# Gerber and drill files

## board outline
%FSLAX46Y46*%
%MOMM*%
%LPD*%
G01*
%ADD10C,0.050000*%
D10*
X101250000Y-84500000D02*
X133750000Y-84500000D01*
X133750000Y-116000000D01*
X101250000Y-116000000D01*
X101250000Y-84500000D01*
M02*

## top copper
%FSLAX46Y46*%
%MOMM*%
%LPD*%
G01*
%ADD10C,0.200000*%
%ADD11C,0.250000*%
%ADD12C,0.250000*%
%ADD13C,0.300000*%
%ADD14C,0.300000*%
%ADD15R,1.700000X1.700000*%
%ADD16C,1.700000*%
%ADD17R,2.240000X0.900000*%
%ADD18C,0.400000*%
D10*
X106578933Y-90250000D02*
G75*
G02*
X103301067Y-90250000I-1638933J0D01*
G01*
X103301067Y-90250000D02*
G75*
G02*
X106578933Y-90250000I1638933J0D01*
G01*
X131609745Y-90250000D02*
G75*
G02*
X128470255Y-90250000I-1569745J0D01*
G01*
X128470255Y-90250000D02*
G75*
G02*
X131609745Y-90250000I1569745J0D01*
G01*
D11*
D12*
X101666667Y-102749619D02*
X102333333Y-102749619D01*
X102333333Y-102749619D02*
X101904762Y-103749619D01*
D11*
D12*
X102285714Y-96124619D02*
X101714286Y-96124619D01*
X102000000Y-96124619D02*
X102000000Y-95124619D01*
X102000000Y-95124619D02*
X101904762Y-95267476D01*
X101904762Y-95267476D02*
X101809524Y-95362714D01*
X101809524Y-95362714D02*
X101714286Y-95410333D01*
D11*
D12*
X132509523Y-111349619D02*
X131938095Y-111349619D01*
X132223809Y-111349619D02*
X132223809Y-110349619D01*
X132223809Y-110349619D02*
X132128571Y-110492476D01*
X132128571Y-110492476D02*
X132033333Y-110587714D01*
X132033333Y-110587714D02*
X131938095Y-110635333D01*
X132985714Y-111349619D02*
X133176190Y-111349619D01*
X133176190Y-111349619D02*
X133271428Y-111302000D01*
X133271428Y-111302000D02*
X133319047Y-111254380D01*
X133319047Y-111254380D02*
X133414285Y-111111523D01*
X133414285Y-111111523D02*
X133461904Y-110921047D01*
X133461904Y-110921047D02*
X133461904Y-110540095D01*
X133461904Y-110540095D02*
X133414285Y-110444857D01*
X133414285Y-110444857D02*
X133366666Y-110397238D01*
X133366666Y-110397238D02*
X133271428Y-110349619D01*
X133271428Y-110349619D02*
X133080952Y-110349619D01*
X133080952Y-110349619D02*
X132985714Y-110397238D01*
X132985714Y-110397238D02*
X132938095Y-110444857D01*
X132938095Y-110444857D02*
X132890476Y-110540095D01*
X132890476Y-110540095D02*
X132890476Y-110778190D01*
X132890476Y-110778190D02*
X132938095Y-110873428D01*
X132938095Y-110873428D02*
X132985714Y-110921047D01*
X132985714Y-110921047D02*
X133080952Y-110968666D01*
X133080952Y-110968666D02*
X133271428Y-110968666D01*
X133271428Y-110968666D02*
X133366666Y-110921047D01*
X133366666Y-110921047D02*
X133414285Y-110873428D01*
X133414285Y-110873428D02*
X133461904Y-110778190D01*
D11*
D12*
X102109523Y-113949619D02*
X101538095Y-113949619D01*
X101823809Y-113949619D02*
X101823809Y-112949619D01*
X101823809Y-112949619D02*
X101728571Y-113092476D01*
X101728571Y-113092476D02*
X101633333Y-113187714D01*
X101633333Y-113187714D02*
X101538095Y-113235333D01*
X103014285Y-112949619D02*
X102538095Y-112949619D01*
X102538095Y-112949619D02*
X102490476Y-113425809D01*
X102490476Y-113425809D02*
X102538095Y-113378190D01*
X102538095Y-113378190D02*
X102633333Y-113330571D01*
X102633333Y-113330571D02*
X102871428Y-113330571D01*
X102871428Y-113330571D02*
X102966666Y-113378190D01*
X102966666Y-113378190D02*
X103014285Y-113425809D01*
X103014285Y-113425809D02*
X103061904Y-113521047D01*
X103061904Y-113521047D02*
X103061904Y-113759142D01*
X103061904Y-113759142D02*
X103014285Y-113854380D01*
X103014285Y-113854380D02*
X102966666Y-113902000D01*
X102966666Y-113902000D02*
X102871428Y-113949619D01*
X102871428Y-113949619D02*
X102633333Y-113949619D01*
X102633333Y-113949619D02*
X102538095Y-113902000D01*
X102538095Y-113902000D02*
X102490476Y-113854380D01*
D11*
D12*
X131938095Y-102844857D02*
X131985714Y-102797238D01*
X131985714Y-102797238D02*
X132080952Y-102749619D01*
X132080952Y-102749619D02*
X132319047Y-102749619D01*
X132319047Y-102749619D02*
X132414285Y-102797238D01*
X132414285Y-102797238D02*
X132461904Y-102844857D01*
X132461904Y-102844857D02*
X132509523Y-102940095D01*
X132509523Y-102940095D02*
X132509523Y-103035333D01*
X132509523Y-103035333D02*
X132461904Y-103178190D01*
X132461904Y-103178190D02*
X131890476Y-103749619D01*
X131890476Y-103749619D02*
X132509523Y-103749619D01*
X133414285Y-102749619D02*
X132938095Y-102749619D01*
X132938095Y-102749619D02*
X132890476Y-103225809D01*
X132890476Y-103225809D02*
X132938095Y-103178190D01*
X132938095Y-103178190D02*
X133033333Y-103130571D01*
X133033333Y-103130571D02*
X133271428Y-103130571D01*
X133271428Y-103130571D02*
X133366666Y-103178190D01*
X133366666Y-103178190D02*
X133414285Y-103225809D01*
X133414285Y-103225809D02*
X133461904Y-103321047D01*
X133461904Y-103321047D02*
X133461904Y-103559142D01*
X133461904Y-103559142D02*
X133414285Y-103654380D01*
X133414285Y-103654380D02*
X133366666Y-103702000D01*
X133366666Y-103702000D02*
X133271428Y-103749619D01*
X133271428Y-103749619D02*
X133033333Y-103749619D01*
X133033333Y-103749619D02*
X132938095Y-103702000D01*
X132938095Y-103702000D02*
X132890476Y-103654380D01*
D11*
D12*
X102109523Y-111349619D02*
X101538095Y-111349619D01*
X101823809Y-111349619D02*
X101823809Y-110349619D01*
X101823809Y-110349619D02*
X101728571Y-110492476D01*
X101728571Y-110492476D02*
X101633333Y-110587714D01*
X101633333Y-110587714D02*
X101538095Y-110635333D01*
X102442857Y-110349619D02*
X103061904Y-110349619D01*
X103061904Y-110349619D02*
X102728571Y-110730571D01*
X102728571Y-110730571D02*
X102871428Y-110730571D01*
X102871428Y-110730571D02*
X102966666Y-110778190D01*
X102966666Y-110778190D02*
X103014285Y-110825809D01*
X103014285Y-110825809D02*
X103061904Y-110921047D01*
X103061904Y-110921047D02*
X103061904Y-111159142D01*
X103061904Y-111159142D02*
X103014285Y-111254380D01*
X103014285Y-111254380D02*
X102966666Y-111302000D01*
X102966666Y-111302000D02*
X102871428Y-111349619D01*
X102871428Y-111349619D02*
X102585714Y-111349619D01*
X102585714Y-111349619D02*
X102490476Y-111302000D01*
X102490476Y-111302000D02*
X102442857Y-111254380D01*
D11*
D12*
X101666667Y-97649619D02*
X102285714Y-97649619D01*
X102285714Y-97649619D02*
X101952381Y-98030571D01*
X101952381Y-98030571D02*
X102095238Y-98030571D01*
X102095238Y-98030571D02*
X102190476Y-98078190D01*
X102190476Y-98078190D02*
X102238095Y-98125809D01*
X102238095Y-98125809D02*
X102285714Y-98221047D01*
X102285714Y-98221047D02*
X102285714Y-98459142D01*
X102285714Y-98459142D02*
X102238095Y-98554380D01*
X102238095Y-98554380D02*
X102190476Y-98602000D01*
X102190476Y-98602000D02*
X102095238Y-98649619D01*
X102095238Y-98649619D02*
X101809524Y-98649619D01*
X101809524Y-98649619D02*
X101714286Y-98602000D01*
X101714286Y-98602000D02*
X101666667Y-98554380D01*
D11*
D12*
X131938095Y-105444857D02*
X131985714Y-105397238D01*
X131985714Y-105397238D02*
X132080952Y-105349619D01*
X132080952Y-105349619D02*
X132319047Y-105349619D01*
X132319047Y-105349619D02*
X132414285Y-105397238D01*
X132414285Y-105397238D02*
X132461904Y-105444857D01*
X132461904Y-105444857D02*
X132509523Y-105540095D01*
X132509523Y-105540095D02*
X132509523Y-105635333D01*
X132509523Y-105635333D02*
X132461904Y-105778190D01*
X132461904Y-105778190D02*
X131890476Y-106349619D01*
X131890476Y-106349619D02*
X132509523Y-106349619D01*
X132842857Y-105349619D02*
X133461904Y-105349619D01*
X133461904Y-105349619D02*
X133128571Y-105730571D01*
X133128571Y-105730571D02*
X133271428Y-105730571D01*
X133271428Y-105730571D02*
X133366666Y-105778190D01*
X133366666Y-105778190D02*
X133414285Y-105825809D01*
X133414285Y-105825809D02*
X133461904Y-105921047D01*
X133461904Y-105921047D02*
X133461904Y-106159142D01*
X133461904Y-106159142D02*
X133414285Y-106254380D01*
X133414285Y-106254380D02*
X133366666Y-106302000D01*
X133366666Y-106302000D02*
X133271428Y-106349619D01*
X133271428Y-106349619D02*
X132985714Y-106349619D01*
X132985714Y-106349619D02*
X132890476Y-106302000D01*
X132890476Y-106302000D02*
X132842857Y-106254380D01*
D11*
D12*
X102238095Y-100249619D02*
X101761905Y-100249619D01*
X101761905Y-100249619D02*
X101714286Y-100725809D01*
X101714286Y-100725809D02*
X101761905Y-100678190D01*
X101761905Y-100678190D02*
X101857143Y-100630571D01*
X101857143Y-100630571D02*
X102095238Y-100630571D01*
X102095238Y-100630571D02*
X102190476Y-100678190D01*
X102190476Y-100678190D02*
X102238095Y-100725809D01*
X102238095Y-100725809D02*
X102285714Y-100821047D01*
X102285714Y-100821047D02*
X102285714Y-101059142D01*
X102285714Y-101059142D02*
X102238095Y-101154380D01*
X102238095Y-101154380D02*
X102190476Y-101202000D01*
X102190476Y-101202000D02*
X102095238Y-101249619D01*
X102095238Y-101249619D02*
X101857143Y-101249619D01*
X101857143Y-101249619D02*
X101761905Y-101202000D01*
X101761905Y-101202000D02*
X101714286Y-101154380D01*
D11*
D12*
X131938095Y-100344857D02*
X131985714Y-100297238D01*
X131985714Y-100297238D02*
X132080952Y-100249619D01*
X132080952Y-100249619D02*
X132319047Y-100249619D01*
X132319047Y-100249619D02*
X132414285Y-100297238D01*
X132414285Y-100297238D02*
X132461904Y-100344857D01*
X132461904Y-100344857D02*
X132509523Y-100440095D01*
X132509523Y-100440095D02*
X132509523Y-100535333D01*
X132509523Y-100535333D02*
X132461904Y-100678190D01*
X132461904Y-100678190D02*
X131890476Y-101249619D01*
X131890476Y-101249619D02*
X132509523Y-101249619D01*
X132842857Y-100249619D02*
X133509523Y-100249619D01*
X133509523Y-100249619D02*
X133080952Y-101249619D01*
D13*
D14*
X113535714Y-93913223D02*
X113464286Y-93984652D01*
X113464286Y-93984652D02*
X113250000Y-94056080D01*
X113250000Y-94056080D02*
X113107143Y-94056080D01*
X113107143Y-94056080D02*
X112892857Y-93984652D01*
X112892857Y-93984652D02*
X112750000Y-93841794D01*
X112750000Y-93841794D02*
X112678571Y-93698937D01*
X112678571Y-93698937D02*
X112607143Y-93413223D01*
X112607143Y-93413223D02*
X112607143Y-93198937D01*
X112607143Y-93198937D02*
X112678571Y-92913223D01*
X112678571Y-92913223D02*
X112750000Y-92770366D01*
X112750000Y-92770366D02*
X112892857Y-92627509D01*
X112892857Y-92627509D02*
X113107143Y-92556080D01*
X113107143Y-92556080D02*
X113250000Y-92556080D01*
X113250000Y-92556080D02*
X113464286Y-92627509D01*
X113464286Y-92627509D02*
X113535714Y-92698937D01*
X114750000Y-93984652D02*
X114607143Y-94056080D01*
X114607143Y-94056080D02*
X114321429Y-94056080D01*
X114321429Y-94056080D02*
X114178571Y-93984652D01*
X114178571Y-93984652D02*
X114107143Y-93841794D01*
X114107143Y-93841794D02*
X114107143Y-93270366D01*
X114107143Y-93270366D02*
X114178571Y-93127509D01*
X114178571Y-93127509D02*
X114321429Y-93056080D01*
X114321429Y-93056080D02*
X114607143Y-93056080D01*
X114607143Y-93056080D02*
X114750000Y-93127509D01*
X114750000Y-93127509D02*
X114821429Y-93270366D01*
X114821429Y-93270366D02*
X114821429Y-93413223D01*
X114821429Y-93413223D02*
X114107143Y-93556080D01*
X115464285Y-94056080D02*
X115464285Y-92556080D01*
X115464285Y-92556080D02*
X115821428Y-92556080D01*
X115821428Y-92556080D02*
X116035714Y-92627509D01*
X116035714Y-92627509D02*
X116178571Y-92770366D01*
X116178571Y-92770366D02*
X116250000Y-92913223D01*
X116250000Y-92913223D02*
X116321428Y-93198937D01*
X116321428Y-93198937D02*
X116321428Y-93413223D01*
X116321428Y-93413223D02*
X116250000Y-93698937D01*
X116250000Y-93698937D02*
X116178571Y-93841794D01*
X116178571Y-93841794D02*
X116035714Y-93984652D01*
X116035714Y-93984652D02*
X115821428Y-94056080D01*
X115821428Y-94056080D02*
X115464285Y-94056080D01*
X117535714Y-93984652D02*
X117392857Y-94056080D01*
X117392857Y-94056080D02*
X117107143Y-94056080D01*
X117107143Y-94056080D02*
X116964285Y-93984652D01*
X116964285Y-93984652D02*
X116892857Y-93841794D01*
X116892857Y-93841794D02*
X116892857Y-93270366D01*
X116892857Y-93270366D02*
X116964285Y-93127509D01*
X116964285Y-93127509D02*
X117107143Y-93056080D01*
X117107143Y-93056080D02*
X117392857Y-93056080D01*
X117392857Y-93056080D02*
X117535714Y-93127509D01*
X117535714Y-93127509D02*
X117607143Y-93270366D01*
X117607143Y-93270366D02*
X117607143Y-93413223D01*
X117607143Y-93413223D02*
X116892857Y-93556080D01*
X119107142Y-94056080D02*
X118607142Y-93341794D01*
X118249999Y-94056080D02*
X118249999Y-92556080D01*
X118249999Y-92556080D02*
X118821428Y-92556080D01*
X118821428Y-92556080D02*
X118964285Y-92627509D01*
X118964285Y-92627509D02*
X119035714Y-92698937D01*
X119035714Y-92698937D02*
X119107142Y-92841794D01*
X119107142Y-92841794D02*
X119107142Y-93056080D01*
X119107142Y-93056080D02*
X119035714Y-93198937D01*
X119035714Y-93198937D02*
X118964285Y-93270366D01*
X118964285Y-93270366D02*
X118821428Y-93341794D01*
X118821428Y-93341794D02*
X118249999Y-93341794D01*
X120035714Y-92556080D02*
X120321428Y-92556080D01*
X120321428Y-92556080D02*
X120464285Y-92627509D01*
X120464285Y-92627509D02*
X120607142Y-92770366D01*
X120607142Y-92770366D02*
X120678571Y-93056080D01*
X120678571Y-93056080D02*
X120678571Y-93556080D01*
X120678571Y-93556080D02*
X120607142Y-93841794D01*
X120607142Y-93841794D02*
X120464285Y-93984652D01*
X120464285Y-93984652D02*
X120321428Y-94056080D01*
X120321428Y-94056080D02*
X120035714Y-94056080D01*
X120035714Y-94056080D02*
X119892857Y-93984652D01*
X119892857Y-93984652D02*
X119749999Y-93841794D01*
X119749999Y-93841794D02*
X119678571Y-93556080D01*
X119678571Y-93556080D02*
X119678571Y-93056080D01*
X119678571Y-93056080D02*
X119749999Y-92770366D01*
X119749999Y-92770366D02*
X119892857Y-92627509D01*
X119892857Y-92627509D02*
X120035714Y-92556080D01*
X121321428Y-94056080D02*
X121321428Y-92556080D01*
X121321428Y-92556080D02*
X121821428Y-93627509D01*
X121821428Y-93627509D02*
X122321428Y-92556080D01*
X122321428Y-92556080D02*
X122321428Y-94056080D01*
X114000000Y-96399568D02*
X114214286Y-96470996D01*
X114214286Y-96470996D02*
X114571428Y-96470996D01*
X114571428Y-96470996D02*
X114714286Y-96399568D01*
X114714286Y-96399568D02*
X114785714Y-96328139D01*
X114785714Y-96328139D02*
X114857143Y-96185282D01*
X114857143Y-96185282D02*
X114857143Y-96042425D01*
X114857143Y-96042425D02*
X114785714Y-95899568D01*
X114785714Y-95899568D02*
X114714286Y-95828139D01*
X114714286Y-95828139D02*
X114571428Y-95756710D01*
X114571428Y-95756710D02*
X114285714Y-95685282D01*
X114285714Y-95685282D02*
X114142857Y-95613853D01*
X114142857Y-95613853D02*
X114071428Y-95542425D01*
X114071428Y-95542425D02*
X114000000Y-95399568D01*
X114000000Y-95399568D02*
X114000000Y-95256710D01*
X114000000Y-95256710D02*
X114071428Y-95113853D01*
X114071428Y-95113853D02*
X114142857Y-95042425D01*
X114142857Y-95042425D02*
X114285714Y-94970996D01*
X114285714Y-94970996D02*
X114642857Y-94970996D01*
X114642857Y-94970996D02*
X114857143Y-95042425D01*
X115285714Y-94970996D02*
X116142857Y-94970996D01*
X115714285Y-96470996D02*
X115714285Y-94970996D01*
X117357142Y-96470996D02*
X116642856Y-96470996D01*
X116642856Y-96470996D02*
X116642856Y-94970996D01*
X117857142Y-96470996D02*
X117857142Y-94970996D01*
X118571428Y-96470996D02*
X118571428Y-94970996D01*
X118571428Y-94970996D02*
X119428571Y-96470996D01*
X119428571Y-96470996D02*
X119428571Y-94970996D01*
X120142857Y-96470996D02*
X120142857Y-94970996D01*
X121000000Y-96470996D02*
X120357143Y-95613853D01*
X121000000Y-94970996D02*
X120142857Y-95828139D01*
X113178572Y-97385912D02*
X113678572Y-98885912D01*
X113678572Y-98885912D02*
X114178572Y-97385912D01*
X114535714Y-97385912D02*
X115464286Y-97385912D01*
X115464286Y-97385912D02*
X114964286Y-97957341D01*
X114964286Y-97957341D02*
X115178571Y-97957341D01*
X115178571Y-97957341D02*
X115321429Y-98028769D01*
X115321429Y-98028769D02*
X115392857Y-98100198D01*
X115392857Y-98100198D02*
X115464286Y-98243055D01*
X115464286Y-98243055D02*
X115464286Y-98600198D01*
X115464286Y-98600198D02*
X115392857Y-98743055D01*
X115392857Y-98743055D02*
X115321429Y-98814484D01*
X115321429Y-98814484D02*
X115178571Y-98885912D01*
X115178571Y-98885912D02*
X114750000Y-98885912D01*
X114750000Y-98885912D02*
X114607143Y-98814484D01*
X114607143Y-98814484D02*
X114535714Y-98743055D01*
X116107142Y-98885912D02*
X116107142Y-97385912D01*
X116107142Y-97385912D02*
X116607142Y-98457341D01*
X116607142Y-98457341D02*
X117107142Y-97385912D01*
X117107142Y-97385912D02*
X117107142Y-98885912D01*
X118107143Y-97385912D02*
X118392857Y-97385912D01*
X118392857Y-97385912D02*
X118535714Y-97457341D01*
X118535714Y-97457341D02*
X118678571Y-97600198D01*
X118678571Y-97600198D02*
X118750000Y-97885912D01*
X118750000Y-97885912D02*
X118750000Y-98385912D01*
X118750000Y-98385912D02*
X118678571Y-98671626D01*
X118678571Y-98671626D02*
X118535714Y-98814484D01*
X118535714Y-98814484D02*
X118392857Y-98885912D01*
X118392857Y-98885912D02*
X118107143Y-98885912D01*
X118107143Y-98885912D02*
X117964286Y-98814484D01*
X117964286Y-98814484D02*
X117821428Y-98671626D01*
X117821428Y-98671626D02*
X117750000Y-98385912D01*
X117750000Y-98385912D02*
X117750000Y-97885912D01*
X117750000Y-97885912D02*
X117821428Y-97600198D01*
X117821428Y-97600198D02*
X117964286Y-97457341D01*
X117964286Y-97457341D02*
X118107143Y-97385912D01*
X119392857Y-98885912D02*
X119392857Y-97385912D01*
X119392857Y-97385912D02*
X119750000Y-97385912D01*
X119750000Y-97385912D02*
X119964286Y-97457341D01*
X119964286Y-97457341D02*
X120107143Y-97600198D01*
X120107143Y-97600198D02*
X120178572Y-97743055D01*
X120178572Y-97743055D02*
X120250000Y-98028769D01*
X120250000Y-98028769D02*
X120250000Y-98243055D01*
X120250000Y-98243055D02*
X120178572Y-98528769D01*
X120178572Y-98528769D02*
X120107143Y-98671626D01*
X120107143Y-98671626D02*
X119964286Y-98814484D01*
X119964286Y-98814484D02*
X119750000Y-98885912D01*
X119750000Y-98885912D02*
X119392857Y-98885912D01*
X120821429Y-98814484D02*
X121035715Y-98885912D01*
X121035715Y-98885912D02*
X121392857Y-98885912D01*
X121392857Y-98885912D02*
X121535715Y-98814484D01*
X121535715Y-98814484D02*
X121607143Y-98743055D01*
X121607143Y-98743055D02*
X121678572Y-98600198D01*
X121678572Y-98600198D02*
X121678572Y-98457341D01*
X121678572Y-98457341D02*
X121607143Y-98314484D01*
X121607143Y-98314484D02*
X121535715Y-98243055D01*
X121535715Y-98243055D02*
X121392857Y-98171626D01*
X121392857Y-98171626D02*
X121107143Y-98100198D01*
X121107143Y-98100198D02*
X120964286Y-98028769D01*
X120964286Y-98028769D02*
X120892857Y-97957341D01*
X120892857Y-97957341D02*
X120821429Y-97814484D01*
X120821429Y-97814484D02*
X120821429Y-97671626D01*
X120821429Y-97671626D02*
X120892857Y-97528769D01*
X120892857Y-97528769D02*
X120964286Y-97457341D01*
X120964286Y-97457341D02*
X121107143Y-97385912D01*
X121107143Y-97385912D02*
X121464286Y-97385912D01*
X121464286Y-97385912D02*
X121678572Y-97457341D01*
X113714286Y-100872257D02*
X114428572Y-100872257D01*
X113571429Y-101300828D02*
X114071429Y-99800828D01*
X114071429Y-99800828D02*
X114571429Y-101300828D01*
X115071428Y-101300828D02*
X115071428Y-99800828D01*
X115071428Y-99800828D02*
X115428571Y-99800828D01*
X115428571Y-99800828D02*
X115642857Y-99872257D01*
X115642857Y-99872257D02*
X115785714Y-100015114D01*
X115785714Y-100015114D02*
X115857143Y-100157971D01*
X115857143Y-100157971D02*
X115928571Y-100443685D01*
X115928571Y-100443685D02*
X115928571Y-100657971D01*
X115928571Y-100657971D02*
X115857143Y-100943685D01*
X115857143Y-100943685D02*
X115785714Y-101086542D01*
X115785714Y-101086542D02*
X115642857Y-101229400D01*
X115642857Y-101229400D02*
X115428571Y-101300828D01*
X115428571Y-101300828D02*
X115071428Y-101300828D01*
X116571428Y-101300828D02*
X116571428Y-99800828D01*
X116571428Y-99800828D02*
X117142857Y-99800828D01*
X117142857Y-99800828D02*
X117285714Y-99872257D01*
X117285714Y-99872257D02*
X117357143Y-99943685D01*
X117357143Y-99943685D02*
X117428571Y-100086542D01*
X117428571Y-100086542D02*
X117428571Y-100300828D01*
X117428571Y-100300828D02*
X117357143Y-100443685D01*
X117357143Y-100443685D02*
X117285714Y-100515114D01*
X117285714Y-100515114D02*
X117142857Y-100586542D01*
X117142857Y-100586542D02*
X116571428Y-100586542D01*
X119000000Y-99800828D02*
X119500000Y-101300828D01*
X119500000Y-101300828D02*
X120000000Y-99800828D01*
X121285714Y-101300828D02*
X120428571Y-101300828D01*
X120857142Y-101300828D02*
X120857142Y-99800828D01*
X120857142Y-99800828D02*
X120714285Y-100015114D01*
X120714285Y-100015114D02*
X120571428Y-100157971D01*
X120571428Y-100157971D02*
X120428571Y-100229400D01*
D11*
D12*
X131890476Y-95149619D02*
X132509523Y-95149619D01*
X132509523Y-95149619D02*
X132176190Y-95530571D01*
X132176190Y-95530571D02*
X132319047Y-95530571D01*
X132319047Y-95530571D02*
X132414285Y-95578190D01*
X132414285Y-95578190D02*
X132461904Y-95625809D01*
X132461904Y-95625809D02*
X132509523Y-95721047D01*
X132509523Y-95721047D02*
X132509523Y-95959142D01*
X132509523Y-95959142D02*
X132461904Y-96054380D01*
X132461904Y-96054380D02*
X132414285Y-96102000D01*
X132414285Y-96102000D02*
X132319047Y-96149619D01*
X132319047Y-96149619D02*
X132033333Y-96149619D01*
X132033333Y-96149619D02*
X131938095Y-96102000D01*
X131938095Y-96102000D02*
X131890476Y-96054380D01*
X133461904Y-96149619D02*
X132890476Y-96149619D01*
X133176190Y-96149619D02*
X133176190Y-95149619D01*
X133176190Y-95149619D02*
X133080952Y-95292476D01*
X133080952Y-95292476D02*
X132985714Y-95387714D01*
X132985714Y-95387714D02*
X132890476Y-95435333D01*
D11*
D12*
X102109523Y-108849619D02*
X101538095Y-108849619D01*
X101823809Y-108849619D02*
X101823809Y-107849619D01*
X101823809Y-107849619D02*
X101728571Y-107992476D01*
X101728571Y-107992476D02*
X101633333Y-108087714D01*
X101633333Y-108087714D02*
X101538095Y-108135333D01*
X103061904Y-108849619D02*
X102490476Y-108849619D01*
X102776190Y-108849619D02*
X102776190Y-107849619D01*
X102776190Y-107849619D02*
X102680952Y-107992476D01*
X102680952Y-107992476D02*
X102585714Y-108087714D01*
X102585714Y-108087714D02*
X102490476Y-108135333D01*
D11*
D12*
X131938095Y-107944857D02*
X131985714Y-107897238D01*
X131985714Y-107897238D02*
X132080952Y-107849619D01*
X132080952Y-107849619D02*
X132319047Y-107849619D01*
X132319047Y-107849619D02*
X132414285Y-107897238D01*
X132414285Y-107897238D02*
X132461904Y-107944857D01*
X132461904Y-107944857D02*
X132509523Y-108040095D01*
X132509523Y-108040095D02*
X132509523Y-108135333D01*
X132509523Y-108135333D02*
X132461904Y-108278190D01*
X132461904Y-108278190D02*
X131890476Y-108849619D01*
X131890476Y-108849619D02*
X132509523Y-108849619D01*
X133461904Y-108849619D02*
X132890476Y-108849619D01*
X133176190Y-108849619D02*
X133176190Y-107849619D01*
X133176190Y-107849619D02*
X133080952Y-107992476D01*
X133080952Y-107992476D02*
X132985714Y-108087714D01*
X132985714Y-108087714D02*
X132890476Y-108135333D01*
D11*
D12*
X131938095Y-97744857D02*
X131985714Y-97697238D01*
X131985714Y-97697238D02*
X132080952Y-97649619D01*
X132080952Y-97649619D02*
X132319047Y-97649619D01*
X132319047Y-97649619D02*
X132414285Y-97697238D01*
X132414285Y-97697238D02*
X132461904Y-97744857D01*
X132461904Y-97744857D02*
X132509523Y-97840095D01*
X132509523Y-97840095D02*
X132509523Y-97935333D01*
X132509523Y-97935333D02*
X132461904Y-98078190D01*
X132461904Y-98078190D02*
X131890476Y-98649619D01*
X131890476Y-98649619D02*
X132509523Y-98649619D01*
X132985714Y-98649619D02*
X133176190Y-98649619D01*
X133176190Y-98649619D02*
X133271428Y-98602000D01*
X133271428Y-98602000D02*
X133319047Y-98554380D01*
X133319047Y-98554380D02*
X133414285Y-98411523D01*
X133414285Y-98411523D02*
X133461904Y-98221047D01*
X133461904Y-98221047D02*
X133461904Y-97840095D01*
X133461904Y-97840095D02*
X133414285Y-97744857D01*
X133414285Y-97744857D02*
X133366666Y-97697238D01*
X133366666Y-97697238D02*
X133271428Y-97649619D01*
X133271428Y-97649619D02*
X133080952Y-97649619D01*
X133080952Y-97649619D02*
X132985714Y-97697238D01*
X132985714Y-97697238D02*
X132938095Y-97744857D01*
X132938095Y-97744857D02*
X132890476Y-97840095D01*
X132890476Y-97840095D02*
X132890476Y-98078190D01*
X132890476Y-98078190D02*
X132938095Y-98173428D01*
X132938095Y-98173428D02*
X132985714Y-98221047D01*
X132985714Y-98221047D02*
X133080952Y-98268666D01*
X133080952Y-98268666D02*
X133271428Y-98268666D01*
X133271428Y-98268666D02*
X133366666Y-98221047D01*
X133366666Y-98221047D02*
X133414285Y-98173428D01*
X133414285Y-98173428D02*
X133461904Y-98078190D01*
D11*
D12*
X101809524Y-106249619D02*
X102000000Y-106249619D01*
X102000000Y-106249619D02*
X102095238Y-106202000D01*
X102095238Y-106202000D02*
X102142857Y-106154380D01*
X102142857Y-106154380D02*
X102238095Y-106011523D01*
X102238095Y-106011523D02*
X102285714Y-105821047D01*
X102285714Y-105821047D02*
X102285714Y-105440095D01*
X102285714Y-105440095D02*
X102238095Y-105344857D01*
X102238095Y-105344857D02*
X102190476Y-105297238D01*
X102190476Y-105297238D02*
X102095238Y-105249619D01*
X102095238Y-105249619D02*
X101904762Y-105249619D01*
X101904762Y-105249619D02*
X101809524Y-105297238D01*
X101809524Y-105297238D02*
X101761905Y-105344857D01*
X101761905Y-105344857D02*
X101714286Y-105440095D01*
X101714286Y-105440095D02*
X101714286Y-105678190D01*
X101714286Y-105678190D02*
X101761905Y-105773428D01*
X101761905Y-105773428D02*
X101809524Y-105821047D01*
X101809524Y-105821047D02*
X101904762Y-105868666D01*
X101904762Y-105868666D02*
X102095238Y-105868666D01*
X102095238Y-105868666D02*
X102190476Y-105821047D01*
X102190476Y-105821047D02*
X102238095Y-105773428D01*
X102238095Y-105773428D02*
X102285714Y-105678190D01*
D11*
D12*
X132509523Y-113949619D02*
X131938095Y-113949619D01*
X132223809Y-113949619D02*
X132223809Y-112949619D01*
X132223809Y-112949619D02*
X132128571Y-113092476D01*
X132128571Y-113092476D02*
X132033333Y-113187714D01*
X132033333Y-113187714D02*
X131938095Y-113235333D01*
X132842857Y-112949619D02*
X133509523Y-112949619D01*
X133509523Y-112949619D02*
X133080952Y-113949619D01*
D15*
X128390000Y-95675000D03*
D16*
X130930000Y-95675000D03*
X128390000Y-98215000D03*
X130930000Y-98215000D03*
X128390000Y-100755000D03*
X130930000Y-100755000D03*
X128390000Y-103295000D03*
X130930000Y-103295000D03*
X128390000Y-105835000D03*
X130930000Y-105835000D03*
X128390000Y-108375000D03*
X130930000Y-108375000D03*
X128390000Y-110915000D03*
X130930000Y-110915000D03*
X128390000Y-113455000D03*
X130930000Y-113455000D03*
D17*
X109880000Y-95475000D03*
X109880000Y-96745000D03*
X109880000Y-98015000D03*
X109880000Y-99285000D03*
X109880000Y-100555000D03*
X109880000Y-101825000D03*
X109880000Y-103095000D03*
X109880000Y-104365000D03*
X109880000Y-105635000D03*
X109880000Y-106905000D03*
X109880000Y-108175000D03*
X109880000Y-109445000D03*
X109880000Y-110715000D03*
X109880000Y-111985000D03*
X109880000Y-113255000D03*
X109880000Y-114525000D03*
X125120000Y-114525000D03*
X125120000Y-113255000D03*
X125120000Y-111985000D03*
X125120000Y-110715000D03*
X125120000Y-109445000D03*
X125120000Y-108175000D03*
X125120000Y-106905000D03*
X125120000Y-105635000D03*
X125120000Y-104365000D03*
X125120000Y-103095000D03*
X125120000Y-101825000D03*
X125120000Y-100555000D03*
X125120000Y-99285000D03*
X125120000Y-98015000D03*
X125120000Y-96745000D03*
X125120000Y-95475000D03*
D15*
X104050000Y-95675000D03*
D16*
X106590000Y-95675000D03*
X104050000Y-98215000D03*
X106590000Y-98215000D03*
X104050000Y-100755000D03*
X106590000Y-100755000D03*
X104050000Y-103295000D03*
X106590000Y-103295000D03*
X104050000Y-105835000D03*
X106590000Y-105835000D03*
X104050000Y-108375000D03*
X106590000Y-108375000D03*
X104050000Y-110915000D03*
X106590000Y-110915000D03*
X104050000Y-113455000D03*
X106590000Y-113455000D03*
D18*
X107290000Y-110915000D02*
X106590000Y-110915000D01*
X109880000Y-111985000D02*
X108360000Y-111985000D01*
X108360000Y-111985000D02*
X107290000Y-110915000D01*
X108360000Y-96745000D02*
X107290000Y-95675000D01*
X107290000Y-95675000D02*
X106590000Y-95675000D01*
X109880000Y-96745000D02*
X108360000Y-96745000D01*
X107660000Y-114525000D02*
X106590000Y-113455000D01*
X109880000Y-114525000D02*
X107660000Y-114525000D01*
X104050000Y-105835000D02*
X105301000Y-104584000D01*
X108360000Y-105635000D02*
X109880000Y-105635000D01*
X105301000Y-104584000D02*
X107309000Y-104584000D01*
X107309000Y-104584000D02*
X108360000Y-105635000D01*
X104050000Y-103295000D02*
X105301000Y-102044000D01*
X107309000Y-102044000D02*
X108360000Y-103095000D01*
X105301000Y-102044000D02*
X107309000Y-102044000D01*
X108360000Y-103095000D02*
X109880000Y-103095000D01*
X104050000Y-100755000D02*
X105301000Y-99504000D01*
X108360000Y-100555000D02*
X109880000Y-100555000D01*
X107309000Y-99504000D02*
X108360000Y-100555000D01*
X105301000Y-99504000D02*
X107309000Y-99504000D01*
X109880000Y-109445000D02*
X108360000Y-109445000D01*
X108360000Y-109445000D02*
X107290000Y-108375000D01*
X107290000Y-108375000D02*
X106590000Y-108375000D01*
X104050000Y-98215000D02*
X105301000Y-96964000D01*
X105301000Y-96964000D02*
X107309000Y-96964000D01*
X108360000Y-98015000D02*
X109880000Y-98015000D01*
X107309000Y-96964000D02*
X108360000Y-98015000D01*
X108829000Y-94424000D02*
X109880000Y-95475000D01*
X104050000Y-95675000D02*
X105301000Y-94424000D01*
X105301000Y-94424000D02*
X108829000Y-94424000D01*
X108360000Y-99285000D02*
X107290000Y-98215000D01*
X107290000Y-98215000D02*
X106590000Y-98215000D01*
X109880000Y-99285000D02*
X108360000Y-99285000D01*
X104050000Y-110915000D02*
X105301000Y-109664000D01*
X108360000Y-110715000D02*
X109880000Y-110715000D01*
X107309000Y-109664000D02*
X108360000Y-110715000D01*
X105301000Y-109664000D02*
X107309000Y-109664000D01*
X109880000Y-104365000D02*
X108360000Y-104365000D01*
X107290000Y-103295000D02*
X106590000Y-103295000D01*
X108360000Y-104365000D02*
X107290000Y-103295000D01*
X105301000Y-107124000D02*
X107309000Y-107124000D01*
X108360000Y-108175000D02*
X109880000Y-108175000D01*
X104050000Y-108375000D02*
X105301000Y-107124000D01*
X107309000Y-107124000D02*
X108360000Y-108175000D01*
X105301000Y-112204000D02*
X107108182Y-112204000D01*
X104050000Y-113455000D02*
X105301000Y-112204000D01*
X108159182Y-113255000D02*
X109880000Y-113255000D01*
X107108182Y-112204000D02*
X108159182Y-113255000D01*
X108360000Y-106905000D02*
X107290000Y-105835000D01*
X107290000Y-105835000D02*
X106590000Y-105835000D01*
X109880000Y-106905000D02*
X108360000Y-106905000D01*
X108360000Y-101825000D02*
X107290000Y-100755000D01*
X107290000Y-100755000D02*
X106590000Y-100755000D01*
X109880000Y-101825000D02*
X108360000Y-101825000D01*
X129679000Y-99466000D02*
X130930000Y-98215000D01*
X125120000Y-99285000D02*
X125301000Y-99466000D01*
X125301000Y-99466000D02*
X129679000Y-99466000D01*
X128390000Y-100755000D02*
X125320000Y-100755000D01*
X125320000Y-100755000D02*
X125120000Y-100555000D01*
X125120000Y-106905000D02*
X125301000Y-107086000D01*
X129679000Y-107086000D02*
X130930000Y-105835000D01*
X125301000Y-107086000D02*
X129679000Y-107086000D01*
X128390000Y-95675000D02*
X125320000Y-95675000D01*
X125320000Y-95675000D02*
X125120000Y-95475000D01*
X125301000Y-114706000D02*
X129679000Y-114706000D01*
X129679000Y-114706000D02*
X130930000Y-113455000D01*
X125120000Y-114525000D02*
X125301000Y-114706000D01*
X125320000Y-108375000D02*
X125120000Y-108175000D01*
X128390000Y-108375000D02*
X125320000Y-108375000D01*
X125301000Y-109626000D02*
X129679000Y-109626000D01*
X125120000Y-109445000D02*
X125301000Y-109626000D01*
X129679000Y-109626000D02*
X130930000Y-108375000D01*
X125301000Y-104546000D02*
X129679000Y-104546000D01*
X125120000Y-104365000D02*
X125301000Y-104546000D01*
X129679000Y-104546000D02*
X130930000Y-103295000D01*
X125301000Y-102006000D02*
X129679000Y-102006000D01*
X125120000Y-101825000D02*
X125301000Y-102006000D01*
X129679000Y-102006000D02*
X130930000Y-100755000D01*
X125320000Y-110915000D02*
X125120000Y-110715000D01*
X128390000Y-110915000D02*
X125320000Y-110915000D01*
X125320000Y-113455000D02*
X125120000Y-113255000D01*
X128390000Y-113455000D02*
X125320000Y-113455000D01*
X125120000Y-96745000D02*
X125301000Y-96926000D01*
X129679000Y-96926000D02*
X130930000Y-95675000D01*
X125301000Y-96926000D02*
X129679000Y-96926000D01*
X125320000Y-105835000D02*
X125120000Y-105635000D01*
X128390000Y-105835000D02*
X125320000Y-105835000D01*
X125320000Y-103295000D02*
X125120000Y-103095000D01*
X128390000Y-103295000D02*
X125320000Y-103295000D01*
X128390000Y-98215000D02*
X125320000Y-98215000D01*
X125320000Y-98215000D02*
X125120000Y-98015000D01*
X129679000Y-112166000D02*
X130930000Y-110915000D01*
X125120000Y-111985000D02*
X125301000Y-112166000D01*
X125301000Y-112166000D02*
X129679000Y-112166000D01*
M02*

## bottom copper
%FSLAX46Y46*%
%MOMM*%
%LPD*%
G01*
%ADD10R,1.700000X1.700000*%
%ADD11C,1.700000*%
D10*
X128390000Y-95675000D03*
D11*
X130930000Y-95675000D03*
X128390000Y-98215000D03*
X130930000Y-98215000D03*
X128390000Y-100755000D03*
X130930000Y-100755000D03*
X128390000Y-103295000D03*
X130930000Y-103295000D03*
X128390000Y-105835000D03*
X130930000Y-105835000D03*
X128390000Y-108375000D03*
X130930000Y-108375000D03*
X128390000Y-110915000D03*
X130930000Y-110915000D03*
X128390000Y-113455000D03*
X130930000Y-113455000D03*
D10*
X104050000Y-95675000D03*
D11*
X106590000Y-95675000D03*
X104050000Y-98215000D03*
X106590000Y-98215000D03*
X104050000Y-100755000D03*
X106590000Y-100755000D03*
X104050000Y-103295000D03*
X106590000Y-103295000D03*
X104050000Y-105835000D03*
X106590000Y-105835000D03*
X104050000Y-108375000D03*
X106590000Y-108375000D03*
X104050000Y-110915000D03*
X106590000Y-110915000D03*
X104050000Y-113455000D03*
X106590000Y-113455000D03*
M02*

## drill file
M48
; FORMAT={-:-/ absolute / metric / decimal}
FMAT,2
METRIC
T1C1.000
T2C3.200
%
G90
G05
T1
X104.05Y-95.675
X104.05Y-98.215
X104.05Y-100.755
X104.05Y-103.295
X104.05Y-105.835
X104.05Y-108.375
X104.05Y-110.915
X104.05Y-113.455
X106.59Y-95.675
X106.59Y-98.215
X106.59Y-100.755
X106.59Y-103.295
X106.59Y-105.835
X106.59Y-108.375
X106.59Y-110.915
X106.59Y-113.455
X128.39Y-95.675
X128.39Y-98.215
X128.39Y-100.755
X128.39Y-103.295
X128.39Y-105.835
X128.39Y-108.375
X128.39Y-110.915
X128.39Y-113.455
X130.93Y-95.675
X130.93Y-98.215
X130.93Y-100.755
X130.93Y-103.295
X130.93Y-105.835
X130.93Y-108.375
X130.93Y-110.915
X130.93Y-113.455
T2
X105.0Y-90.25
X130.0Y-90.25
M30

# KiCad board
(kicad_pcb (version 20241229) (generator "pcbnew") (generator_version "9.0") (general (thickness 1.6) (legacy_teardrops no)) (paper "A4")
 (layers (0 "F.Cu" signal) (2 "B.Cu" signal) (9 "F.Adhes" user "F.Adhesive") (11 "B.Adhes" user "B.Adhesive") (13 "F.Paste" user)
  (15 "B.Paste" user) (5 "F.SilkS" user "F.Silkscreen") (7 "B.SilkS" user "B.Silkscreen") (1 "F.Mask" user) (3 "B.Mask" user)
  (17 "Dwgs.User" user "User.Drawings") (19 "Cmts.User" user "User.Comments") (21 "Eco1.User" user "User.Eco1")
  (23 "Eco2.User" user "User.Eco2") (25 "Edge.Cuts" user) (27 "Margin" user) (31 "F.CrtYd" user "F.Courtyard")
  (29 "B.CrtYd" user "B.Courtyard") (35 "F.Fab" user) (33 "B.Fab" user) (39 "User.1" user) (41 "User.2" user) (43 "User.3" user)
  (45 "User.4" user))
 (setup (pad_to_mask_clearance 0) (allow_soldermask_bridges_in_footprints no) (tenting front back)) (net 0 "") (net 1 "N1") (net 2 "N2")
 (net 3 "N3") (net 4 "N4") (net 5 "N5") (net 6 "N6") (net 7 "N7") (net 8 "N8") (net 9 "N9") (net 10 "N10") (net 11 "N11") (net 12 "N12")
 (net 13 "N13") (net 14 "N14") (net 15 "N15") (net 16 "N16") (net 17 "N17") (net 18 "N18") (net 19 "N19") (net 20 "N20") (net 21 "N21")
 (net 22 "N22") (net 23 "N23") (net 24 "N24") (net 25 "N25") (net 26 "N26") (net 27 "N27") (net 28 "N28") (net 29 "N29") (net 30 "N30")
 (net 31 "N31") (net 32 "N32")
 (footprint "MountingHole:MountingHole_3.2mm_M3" (layer "F.Cu") (at 130 90.25)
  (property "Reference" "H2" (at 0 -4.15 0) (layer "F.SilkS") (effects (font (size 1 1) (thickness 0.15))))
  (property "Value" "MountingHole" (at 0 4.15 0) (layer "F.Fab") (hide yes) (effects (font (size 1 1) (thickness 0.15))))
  (pad "" np_thru_hole circle (at 0 0) (size 3.2 3.2) (drill 3.2) (layers "*.Cu" "*.Mask")))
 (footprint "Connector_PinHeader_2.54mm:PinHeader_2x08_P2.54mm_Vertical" (layer "F.Cu") (at 128.39 95.675)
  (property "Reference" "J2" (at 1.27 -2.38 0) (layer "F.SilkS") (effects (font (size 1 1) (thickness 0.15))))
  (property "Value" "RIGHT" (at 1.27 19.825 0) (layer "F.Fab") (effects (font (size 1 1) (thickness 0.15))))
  (pad "1" thru_hole rect (at 0 0) (size 1.7 1.7) (drill 1) (layers "*.Cu" "*.Mask") (remove_unused_layers no) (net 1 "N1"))
  (pad "2" thru_hole circle (at 2.54 0) (size 1.7 1.7) (drill 1) (layers "*.Cu" "*.Mask") (remove_unused_layers no) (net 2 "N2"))
  (pad "3" thru_hole circle (at 0 2.54) (size 1.7 1.7) (drill 1) (layers "*.Cu" "*.Mask") (remove_unused_layers no) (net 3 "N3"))
  (pad "4" thru_hole circle (at 2.54 2.54) (size 1.7 1.7) (drill 1) (layers "*.Cu" "*.Mask") (remove_unused_layers no) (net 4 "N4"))
  (pad "5" thru_hole circle (at 0 5.08) (size 1.7 1.7) (drill 1) (layers "*.Cu" "*.Mask") (remove_unused_layers no) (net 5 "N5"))
  (pad "6" thru_hole circle (at 2.54 5.08) (size 1.7 1.7) (drill 1) (layers "*.Cu" "*.Mask") (remove_unused_layers no) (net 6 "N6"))
  (pad "7" thru_hole circle (at 0 7.62) (size 1.7 1.7) (drill 1) (layers "*.Cu" "*.Mask") (remove_unused_layers no) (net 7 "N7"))
  (pad "8" thru_hole circle (at 2.54 7.62) (size 1.7 1.7) (drill 1) (layers "*.Cu" "*.Mask") (remove_unused_layers no) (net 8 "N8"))
  (pad "9" thru_hole circle (at 0 10.16) (size 1.7 1.7) (drill 1) (layers "*.Cu" "*.Mask") (remove_unused_layers no) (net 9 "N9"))
  (pad "10" thru_hole circle (at 2.54 10.16) (size 1.7 1.7) (drill 1) (layers "*.Cu" "*.Mask") (remove_unused_layers no) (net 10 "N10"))
  (pad "11" thru_hole circle (at 0 12.7) (size 1.7 1.7) (drill 1) (layers "*.Cu" "*.Mask") (remove_unused_layers no) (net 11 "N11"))
  (pad "12" thru_hole circle (at 2.54 12.7) (size 1.7 1.7) (drill 1) (layers "*.Cu" "*.Mask") (remove_unused_layers no) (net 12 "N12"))
  (pad "13" thru_hole circle (at 0 15.24) (size 1.7 1.7) (drill 1) (layers "*.Cu" "*.Mask") (remove_unused_layers no) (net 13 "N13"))
  (pad "14" thru_hole circle (at 2.54 15.24) (size 1.7 1.7) (drill 1) (layers "*.Cu" "*.Mask") (remove_unused_layers no) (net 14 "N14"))
  (pad "15" thru_hole circle (at 0 17.78) (size 1.7 1.7) (drill 1) (layers "*.Cu" "*.Mask") (remove_unused_layers no) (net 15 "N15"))
  (pad "16" thru_hole circle (at 2.54 17.78) (size 1.7 1.7) (drill 1) (layers "*.Cu" "*.Mask") (remove_unused_layers no) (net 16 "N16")))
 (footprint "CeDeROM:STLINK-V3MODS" (layer "F.Cu") (at 117.5 105)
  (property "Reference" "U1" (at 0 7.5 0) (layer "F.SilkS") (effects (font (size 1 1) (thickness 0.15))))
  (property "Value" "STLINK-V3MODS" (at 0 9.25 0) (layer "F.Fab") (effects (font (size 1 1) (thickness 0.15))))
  (pad "1" smd rect (at -7.62 -9.525 270) (size 0.9 2.24) (layers "F.Cu" "F.Mask" "F.Paste") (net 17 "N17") (thermal_bridge_angle 45))
  (pad "2" smd rect (at -7.62 -8.255 270) (size 0.9 2.24) (layers "F.Cu" "F.Mask" "F.Paste") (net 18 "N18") (thermal_bridge_angle 45))
  (pad "3" smd rect (at -7.62 -6.985 270) (size 0.9 2.24) (layers "F.Cu" "F.Mask" "F.Paste") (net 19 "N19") (thermal_bridge_angle 45))
  (pad "4" smd rect (at -7.62 -5.715 270) (size 0.9 2.24) (layers "F.Cu" "F.Mask" "F.Paste") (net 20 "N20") (thermal_bridge_angle 45))
  (pad "5" smd rect (at -7.62 -4.445 270) (size 0.9 2.24) (layers "F.Cu" "F.Mask" "F.Paste") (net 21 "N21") (thermal_bridge_angle 45))
  (pad "6" smd rect (at -7.62 -3.175 270) (size 0.9 2.24) (layers "F.Cu" "F.Mask" "F.Paste") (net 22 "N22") (thermal_bridge_angle 45))
  (pad "7" smd rect (at -7.62 -1.905 270) (size 0.9 2.24) (layers "F.Cu" "F.Mask" "F.Paste") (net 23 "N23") (thermal_bridge_angle 45))
  (pad "8" smd rect (at -7.62 -0.635 270) (size 0.9 2.24) (layers "F.Cu" "F.Mask" "F.Paste") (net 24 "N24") (thermal_bridge_angle 45))
  (pad "9" smd rect (at -7.62 0.635 270) (size 0.9 2.24) (layers "F.Cu" "F.Mask" "F.Paste") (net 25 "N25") (thermal_bridge_angle 45))
  (pad "10" smd rect (at -7.62 1.905 270) (size 0.9 2.24) (layers "F.Cu" "F.Mask" "F.Paste") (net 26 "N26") (thermal_bridge_angle 45))
  (pad "11" smd rect (at -7.62 3.175 270) (size 0.9 2.24) (layers "F.Cu" "F.Mask" "F.Paste") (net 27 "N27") (thermal_bridge_angle 45))
  (pad "12" smd rect (at -7.62 4.445 270) (size 0.9 2.24) (layers "F.Cu" "F.Mask" "F.Paste") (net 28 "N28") (thermal_bridge_angle 45))
  (pad "13" smd rect (at -7.62 5.715 270) (size 0.9 2.24) (layers "F.Cu" "F.Mask" "F.Paste") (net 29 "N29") (thermal_bridge_angle 45))
  (pad "14" smd rect (at -7.62 6.985 270) (size 0.9 2.24) (layers "F.Cu" "F.Mask" "F.Paste") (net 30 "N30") (thermal_bridge_angle 45))
  (pad "15" smd rect (at -7.62 8.255 270) (size 0.9 2.24) (layers "F.Cu" "F.Mask" "F.Paste") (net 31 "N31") (thermal_bridge_angle 45))
  (pad "16" smd rect (at -7.62 9.525 270) (size 0.9 2.24) (layers "F.Cu" "F.Mask" "F.Paste") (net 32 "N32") (thermal_bridge_angle 45))
  (pad "17" smd rect (at 7.62 9.525 270) (size 0.9 2.24) (layers "F.Cu" "F.Mask" "F.Paste") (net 16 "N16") (thermal_bridge_angle 45))
  (pad "18" smd rect (at 7.62 8.255 270) (size 0.9 2.24) (layers "F.Cu" "F.Mask" "F.Paste") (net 15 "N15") (thermal_bridge_angle 45))
  (pad "19" smd rect (at 7.62 6.985 270) (size 0.9 2.24) (layers "F.Cu" "F.Mask" "F.Paste") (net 14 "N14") (thermal_bridge_angle 45))
  (pad "20" smd rect (at 7.62 5.715 270) (size 0.9 2.24) (layers "F.Cu" "F.Mask" "F.Paste") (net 13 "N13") (thermal_bridge_angle 45))
  (pad "21" smd rect (at 7.62 4.445 270) (size 0.9 2.24) (layers "F.Cu" "F.Mask" "F.Paste") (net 12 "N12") (thermal_bridge_angle 45))
  (pad "22" smd rect (at 7.62 3.175 270) (size 0.9 2.24) (layers "F.Cu" "F.Mask" "F.Paste") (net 11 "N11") (thermal_bridge_angle 45))
  (pad "23" smd rect (at 7.62 1.905 270) (size 0.9 2.24) (layers "F.Cu" "F.Mask" "F.Paste") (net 10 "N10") (thermal_bridge_angle 45))
  (pad "24" smd rect (at 7.62 0.635 270) (size 0.9 2.24) (layers "F.Cu" "F.Mask" "F.Paste") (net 9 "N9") (thermal_bridge_angle 45))
  (pad "25" smd rect (at 7.62 -0.635 270) (size 0.9 2.24) (layers "F.Cu" "F.Mask" "F.Paste") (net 8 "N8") (thermal_bridge_angle 45))
  (pad "26" smd rect (at 7.62 -1.905 270) (size 0.9 2.24) (layers "F.Cu" "F.Mask" "F.Paste") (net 7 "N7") (thermal_bridge_angle 45))
  (pad "27" smd rect (at 7.62 -3.175 270) (size 0.9 2.24) (layers "F.Cu" "F.Mask" "F.Paste") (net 6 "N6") (thermal_bridge_angle 45))
  (pad "28" smd rect (at 7.62 -4.445 270) (size 0.9 2.24) (layers "F.Cu" "F.Mask" "F.Paste") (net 5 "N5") (thermal_bridge_angle 45))
  (pad "29" smd rect (at 7.62 -5.715 270) (size 0.9 2.24) (layers "F.Cu" "F.Mask" "F.Paste") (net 4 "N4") (thermal_bridge_angle 45))
  (pad "30" smd rect (at 7.62 -6.985 270) (size 0.9 2.24) (layers "F.Cu" "F.Mask" "F.Paste") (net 3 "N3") (thermal_bridge_angle 45))
  (pad "31" smd rect (at 7.62 -8.255 270) (size 0.9 2.24) (layers "F.Cu" "F.Mask" "F.Paste") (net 2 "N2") (thermal_bridge_angle 45))
  (pad "32" smd rect (at 7.62 -9.525 270) (size 0.9 2.24) (layers "F.Cu" "F.Mask" "F.Paste") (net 1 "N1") (thermal_bridge_angle 45)))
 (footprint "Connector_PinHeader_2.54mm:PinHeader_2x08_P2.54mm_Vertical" (layer "F.Cu") (at 104.05 95.675)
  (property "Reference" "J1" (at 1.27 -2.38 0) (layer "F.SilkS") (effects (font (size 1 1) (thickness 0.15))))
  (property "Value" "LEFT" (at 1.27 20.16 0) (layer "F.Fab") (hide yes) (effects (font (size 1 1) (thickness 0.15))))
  (pad "1" thru_hole rect (at 0 0) (size 1.7 1.7) (drill 1) (layers "*.Cu" "*.Mask") (remove_unused_layers no) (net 17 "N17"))
  (pad "2" thru_hole circle (at 2.54 0) (size 1.7 1.7) (drill 1) (layers "*.Cu" "*.Mask") (remove_unused_layers no) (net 18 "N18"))
  (pad "3" thru_hole circle (at 0 2.54) (size 1.7 1.7) (drill 1) (layers "*.Cu" "*.Mask") (remove_unused_layers no) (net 19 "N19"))
  (pad "4" thru_hole circle (at 2.54 2.54) (size 1.7 1.7) (drill 1) (layers "*.Cu" "*.Mask") (remove_unused_layers no) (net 20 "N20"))
  (pad "5" thru_hole circle (at 0 5.08) (size 1.7 1.7) (drill 1) (layers "*.Cu" "*.Mask") (remove_unused_layers no) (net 21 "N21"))
  (pad "6" thru_hole circle (at 2.54 5.08) (size 1.7 1.7) (drill 1) (layers "*.Cu" "*.Mask") (remove_unused_layers no) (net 22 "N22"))
  (pad "7" thru_hole circle (at 0 7.62) (size 1.7 1.7) (drill 1) (layers "*.Cu" "*.Mask") (remove_unused_layers no) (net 23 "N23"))
  (pad "8" thru_hole circle (at 2.54 7.62) (size 1.7 1.7) (drill 1) (layers "*.Cu" "*.Mask") (remove_unused_layers no) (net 24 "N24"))
  (pad "9" thru_hole circle (at 0 10.16) (size 1.7 1.7) (drill 1) (layers "*.Cu" "*.Mask") (remove_unused_layers no) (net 25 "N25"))
  (pad "10" thru_hole circle (at 2.54 10.16) (size 1.7 1.7) (drill 1) (layers "*.Cu" "*.Mask") (remove_unused_layers no) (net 26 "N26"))
  (pad "11" thru_hole circle (at 0 12.7) (size 1.7 1.7) (drill 1) (layers "*.Cu" "*.Mask") (remove_unused_layers no) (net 27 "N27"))
  (pad "12" thru_hole circle (at 2.54 12.7) (size 1.7 1.7) (drill 1) (layers "*.Cu" "*.Mask") (remove_unused_layers no) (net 28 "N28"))
  (pad "13" thru_hole circle (at 0 15.24) (size 1.7 1.7) (drill 1) (layers "*.Cu" "*.Mask") (remove_unused_layers no) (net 29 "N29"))
  (pad "14" thru_hole circle (at 2.54 15.24) (size 1.7 1.7) (drill 1) (layers "*.Cu" "*.Mask") (remove_unused_layers no) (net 30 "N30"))
  (pad "15" thru_hole circle (at 0 17.78) (size 1.7 1.7) (drill 1) (layers "*.Cu" "*.Mask") (remove_unused_layers no) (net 31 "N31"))
  (pad "16" thru_hole circle (at 2.54 17.78) (size 1.7 1.7) (drill 1) (layers "*.Cu" "*.Mask") (remove_unused_layers no) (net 32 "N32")))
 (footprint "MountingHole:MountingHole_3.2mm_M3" (layer "F.Cu") (at 105 90.25)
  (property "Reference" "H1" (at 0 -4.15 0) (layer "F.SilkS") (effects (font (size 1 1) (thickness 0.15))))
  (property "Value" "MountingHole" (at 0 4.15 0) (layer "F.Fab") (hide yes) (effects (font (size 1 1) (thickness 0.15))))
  (pad "" np_thru_hole circle (at 0 0) (size 3.2 3.2) (drill 3.2) (layers "*.Cu" "*.Mask")))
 (gr_circle (center 104.94 90.25) (end 106 91.5) (stroke (width 0.2) (type default)) (fill no) (layer "F.Cu"))
 (gr_circle (center 130.04 90.25) (end 131.25 91.25) (stroke (width 0.2) (type default)) (fill no) (layer "F.Cu"))
 (gr_rect (start 101.25 84.5) (end 133.75 116) (stroke (width 0.05) (type default)) (fill no) (layer "Edge.Cuts"))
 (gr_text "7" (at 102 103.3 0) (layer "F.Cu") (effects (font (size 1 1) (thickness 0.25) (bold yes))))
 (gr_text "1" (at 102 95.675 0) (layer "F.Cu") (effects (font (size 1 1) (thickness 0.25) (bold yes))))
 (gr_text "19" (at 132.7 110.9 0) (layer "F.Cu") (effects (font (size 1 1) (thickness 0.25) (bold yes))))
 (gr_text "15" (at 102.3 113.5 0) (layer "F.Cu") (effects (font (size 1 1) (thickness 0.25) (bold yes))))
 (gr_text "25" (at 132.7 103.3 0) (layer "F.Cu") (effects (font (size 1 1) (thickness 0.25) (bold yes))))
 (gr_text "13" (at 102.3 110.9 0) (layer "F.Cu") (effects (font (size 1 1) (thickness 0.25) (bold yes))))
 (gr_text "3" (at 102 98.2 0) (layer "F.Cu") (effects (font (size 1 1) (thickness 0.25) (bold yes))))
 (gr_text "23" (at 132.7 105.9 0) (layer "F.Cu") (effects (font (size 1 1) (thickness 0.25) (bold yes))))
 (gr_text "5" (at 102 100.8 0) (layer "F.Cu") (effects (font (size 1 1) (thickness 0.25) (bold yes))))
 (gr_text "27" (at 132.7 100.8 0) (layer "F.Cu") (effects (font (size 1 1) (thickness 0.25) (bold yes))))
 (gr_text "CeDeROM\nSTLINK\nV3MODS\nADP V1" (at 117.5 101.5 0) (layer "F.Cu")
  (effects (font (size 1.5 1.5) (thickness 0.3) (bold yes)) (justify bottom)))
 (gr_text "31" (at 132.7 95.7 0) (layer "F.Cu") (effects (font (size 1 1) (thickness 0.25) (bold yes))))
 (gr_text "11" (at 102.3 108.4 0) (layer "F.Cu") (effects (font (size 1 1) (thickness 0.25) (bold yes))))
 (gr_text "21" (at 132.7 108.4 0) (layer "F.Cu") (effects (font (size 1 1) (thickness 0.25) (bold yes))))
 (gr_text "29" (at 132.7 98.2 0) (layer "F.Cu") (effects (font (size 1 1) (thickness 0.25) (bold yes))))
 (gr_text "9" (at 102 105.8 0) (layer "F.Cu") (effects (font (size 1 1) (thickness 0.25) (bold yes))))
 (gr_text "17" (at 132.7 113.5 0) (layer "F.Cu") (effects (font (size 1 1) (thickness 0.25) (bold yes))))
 (segment (start 107.29 110.915) (end 106.59 110.915) (width 0.4) (layer "F.Cu") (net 30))
 (segment (start 109.88 111.985) (end 108.36 111.985) (width 0.4) (layer "F.Cu") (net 30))
 (segment (start 108.36 111.985) (end 107.29 110.915) (width 0.4) (layer "F.Cu") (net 30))
 (segment (start 108.36 96.745) (end 107.29 95.675) (width 0.4) (layer "F.Cu") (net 18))
 (segment (start 107.29 95.675) (end 106.59 95.675) (width 0.4) (layer "F.Cu") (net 18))
 (segment (start 109.88 96.745) (end 108.36 96.745) (width 0.4) (layer "F.Cu") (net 18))
 (segment (start 107.66 114.525) (end 106.59 113.455) (width 0.4) (layer "F.Cu") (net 32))
 (segment (start 109.88 114.525) (end 107.66 114.525) (width 0.4) (layer "F.Cu") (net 32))
 (segment (start 104.05 105.835) (end 105.301 104.584) (width 0.4) (layer "F.Cu") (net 25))
 (segment (start 108.36 105.635) (end 109.88 105.635) (width 0.4) (layer "F.Cu") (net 25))
 (segment (start 105.301 104.584) (end 107.309 104.584) (width 0.4) (layer "F.Cu") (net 25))
 (segment (start 107.309 104.584) (end 108.36 105.635) (width 0.4) (layer "F.Cu") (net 25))
 (segment (start 104.05 103.295) (end 105.301 102.044) (width 0.4) (layer "F.Cu") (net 23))
 (segment (start 107.309 102.044) (end 108.36 103.095) (width 0.4) (layer "F.Cu") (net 23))
 (segment (start 105.301 102.044) (end 107.309 102.044) (width 0.4) (layer "F.Cu") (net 23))
 (segment (start 108.36 103.095) (end 109.88 103.095) (width 0.4) (layer "F.Cu") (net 23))
 (segment (start 104.05 100.755) (end 105.301 99.504) (width 0.4) (layer "F.Cu") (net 21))
 (segment (start 108.36 100.555) (end 109.88 100.555) (width 0.4) (layer "F.Cu") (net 21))
 (segment (start 107.309 99.504) (end 108.36 100.555) (width 0.4) (layer "F.Cu") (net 21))
 (segment (start 105.301 99.504) (end 107.309 99.504) (width 0.4) (layer "F.Cu") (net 21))
 (segment (start 109.88 109.445) (end 108.36 109.445) (width 0.4) (layer "F.Cu") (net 28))
 (segment (start 108.36 109.445) (end 107.29 108.375) (width 0.4) (layer "F.Cu") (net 28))
 (segment (start 107.29 108.375) (end 106.59 108.375) (width 0.4) (layer "F.Cu") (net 28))
 (segment (start 104.05 98.215) (end 105.301 96.964) (width 0.4) (layer "F.Cu") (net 19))
 (segment (start 105.301 96.964) (end 107.309 96.964) (width 0.4) (layer "F.Cu") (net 19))
 (segment (start 108.36 98.015) (end 109.88 98.015) (width 0.4) (layer "F.Cu") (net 19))
 (segment (start 107.309 96.964) (end 108.36 98.015) (width 0.4) (layer "F.Cu") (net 19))
 (segment (start 108.829 94.424) (end 109.88 95.475) (width 0.4) (layer "F.Cu") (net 17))
 (segment (start 104.05 95.675) (end 105.301 94.424) (width 0.4) (layer "F.Cu") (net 17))
 (segment (start 105.301 94.424) (end 108.829 94.424) (width 0.4) (layer "F.Cu") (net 17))
 (segment (start 108.36 99.285) (end 107.29 98.215) (width 0.4) (layer "F.Cu") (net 20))
 (segment (start 107.29 98.215) (end 106.59 98.215) (width 0.4) (layer "F.Cu") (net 20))
 (segment (start 109.88 99.285) (end 108.36 99.285) (width 0.4) (layer "F.Cu") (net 20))
 (segment (start 104.05 110.915) (end 105.301 109.664) (width 0.4) (layer "F.Cu") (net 29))
 (segment (start 108.36 110.715) (end 109.88 110.715) (width 0.4) (layer "F.Cu") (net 29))
 (segment (start 107.309 109.664) (end 108.36 110.715) (width 0.4) (layer "F.Cu") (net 29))
 (segment (start 105.301 109.664) (end 107.309 109.664) (width 0.4) (layer "F.Cu") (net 29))
 (segment (start 109.88 104.365) (end 108.36 104.365) (width 0.4) (layer "F.Cu") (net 24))
 (segment (start 107.29 103.295) (end 106.59 103.295) (width 0.4) (layer "F.Cu") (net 24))
 (segment (start 108.36 104.365) (end 107.29 103.295) (width 0.4) (layer "F.Cu") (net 24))
 (segment (start 105.301 107.124) (end 107.309 107.124) (width 0.4) (layer "F.Cu") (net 27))
 (segment (start 108.36 108.175) (end 109.88 108.175) (width 0.4) (layer "F.Cu") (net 27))
 (segment (start 104.05 108.375) (end 105.301 107.124) (width 0.4) (layer "F.Cu") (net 27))
 (segment (start 107.309 107.124) (end 108.36 108.175) (width 0.4) (layer "F.Cu") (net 27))
 (segment (start 105.301 112.204) (end 107.108182 112.204) (width 0.4) (layer "F.Cu") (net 31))
 (segment (start 104.05 113.455) (end 105.301 112.204) (width 0.4) (layer "F.Cu") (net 31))
 (segment (start 108.159182 113.255) (end 109.88 113.255) (width 0.4) (layer "F.Cu") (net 31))
 (segment (start 107.108182 112.204) (end 108.159182 113.255) (width 0.4) (layer "F.Cu") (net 31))
 (segment (start 108.36 106.905) (end 107.29 105.835) (width 0.4) (layer "F.Cu") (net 26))
 (segment (start 107.29 105.835) (end 106.59 105.835) (width 0.4) (layer "F.Cu") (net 26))
 (segment (start 109.88 106.905) (end 108.36 106.905) (width 0.4) (layer "F.Cu") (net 26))
 (segment (start 108.36 101.825) (end 107.29 100.755) (width 0.4) (layer "F.Cu") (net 22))
 (segment (start 107.29 100.755) (end 106.59 100.755) (width 0.4) (layer "F.Cu") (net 22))
 (segment (start 109.88 101.825) (end 108.36 101.825) (width 0.4) (layer "F.Cu") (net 22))
 (segment (start 129.679 99.466) (end 130.93 98.215) (width 0.4) (layer "F.Cu") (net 4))
 (segment (start 125.12 99.285) (end 125.301 99.466) (width 0.4) (layer "F.Cu") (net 4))
 (segment (start 125.301 99.466) (end 129.679 99.466) (width 0.4) (layer "F.Cu") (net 4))
 (segment (start 128.39 100.755) (end 125.32 100.755) (width 0.4) (layer "F.Cu") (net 5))
 (segment (start 125.32 100.755) (end 125.12 100.555) (width 0.4) (layer "F.Cu") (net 5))
 (segment (start 125.12 106.905) (end 125.301 107.086) (width 0.4) (layer "F.Cu") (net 10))
 (segment (start 129.679 107.086) (end 130.93 105.835) (width 0.4) (layer "F.Cu") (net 10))
 (segment (start 125.301 107.086) (end 129.679 107.086) (width 0.4) (layer "F.Cu") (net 10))
 (segment (start 128.39 95.675) (end 125.32 95.675) (width 0.4) (layer "F.Cu") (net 1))
 (segment (start 125.32 95.675) (end 125.12 95.475) (width 0.4) (layer "F.Cu") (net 1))
 (segment (start 125.301 114.706) (end 129.679 114.706) (width 0.4) (layer "F.Cu") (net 16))
 (segment (start 129.679 114.706) (end 130.93 113.455) (width 0.4) (layer "F.Cu") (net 16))
 (segment (start 125.12 114.525) (end 125.301 114.706) (width 0.4) (layer "F.Cu") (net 16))
 (segment (start 125.32 108.375) (end 125.12 108.175) (width 0.4) (layer "F.Cu") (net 11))
 (segment (start 128.39 108.375) (end 125.32 108.375) (width 0.4) (layer "F.Cu") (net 11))
 (segment (start 125.301 109.626) (end 129.679 109.626) (width 0.4) (layer "F.Cu") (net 12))
 (segment (start 125.12 109.445) (end 125.301 109.626) (width 0.4) (layer "F.Cu") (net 12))
 (segment (start 129.679 109.626) (end 130.93 108.375) (width 0.4) (layer "F.Cu") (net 12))
 (segment (start 125.301 104.546) (end 129.679 104.546) (width 0.4) (layer "F.Cu") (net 8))
 (segment (start 125.12 104.365) (end 125.301 104.546) (width 0.4) (layer "F.Cu") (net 8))
 (segment (start 129.679 104.546) (end 130.93 103.295) (width 0.4) (layer "F.Cu") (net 8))
 (segment (start 125.301 102.006) (end 129.679 102.006) (width 0.4) (layer "F.Cu") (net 6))
 (segment (start 125.12 101.825) (end 125.301 102.006) (width 0.4) (layer "F.Cu") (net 6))
 (segment (start 129.679 102.006) (end 130.93 100.755) (width 0.4) (layer "F.Cu") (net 6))
 (segment (start 125.32 110.915) (end 125.12 110.715) (width 0.4) (layer "F.Cu") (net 13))
 (segment (start 128.39 110.915) (end 125.32 110.915) (width 0.4) (layer "F.Cu") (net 13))
 (segment (start 125.32 113.455) (end 125.12 113.255) (width 0.4) (layer "F.Cu") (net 15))
 (segment (start 128.39 113.455) (end 125.32 113.455) (width 0.4) (layer "F.Cu") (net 15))
 (segment (start 125.12 96.745) (end 125.301 96.926) (width 0.4) (layer "F.Cu") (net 2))
 (segment (start 129.679 96.926) (end 130.93 95.675) (width 0.4) (layer "F.Cu") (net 2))
 (segment (start 125.301 96.926) (end 129.679 96.926) (width 0.4) (layer "F.Cu") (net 2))
 (segment (start 125.32 105.835) (end 125.12 105.635) (width 0.4) (layer "F.Cu") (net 9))
 (segment (start 128.39 105.835) (end 125.32 105.835) (width 0.4) (layer "F.Cu") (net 9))
 (segment (start 125.32 103.295) (end 125.12 103.095) (width 0.4) (layer "F.Cu") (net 7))
 (segment (start 128.39 103.295) (end 125.32 103.295) (width 0.4) (layer "F.Cu") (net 7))
 (segment (start 128.39 98.215) (end 125.32 98.215) (width 0.4) (layer "F.Cu") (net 3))
 (segment (start 125.32 98.215) (end 125.12 98.015) (width 0.4) (layer "F.Cu") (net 3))
 (segment (start 129.679 112.166) (end 130.93 110.915) (width 0.4) (layer "F.Cu") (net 14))
 (segment (start 125.12 111.985) (end 125.301 112.166) (width 0.4) (layer "F.Cu") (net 14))
 (segment (start 125.301 112.166) (end 129.679 112.166) (width 0.4) (layer "F.Cu") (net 14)))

